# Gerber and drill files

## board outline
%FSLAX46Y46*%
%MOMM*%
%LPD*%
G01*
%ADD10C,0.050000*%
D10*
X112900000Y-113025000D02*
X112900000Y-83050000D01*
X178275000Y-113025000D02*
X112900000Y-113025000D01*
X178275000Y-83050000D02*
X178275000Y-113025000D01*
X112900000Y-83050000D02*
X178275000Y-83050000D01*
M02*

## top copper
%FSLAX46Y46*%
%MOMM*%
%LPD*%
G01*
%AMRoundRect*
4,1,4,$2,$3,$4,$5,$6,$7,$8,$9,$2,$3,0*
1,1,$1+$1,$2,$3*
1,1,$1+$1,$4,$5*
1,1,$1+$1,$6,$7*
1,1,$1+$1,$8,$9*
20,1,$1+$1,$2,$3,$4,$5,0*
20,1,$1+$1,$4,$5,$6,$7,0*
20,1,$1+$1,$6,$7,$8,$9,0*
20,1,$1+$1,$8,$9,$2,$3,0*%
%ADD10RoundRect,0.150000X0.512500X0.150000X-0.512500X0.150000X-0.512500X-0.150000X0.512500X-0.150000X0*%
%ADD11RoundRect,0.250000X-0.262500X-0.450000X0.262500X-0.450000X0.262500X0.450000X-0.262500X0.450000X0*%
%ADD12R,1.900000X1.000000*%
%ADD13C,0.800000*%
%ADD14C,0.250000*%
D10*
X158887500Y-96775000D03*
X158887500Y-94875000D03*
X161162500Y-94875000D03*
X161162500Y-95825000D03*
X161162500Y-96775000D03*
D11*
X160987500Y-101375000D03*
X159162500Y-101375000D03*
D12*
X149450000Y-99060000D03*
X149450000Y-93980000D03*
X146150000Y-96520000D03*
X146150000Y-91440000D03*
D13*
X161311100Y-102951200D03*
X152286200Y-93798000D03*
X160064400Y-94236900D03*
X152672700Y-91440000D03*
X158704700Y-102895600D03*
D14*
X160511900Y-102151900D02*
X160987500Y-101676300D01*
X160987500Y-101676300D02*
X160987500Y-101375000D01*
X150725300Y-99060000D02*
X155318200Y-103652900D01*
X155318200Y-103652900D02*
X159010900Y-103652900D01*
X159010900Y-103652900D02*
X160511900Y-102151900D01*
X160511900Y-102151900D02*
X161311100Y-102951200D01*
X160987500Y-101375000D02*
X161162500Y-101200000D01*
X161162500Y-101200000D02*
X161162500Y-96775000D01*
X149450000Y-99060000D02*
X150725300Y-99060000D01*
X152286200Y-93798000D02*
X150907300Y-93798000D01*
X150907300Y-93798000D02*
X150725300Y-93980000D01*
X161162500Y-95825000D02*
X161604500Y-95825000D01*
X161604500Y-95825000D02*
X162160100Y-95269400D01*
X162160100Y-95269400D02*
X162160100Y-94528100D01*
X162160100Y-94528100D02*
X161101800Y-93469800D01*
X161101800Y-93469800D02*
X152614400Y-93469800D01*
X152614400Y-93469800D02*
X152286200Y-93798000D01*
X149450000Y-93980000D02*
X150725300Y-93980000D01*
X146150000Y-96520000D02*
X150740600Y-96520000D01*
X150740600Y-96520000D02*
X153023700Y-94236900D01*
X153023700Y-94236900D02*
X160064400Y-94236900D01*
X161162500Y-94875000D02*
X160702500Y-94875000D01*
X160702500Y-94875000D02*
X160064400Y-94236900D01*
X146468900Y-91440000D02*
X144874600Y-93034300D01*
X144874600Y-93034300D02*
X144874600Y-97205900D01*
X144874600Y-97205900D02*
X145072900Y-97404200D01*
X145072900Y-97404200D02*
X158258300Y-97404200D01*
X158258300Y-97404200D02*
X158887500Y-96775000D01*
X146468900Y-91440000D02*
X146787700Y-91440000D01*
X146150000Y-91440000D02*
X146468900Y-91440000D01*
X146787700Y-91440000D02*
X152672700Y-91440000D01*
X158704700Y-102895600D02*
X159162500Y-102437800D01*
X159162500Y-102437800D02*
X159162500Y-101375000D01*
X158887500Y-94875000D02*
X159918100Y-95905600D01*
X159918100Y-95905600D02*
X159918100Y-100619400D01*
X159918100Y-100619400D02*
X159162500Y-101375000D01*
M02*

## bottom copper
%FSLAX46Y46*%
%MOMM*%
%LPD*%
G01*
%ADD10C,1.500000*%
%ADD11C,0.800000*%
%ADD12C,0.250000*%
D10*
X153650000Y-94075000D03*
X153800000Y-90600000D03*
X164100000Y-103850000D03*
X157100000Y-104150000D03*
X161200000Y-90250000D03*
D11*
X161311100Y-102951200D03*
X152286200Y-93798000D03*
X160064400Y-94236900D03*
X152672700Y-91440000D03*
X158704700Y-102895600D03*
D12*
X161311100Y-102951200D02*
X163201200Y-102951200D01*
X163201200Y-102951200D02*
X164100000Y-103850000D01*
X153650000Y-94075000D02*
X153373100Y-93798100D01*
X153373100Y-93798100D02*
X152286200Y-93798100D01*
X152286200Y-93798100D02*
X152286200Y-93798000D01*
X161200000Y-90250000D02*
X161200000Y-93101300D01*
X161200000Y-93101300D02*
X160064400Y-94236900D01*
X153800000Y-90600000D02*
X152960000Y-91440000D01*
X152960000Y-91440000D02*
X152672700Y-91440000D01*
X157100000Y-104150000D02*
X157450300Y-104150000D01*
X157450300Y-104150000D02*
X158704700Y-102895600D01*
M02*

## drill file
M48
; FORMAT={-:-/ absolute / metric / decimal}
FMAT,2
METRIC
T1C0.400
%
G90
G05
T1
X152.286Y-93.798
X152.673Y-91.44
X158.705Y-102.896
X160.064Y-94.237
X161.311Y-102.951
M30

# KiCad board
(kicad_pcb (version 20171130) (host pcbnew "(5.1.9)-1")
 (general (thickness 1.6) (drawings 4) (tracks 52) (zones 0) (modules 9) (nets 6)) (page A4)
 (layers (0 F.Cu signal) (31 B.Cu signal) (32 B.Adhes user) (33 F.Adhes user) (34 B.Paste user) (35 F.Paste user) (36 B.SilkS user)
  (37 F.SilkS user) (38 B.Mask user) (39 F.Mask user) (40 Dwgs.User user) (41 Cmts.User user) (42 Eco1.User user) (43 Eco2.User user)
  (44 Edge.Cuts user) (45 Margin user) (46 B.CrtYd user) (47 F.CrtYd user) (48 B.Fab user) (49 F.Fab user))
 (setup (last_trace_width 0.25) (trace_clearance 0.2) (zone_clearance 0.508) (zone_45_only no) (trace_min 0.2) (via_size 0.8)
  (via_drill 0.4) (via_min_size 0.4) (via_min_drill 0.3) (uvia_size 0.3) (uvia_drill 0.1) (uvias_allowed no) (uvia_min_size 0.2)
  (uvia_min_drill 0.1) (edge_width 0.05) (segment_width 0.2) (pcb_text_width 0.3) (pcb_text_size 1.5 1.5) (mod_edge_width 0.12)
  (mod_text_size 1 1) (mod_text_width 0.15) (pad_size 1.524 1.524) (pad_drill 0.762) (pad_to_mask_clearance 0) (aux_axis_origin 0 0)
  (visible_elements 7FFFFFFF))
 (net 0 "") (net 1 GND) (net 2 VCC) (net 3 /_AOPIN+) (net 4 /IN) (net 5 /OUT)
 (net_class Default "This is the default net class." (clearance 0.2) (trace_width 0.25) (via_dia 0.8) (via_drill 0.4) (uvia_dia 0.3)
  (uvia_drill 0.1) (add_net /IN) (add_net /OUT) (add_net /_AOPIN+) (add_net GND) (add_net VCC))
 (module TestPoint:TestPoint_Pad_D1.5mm (layer B.Cu) (at 153.65 94.075)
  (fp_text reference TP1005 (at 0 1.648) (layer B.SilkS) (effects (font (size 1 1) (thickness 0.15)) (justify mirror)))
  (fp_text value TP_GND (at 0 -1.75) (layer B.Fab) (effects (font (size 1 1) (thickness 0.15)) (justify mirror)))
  (pad 1 smd circle (at 0 0) (size 1.5 1.5) (layers B.Cu B.Mask) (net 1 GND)))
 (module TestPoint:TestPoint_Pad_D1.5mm (layer B.Cu) (at 153.8 90.6)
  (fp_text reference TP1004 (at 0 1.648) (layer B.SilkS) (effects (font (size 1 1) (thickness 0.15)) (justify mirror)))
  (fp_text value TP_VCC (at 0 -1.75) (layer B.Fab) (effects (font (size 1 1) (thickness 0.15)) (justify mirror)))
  (pad 1 smd circle (at 0 0) (size 1.5 1.5) (layers B.Cu B.Mask) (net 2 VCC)))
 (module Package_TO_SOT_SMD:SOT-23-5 (layer F.Cu) (at 160.025 95.825 180)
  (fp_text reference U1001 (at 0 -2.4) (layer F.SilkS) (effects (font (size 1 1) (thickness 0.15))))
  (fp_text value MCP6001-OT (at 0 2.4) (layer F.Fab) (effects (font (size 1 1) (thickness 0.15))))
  (pad 5 smd roundrect (at 1.1375 -0.95 180) (size 1.325 0.6) (layers F.Cu F.Paste F.Mask) (roundrect_rratio 0.25) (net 2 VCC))
  (pad 4 smd roundrect (at 1.1375 0.95 180) (size 1.325 0.6) (layers F.Cu F.Paste F.Mask) (roundrect_rratio 0.25) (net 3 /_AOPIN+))
  (pad 3 smd roundrect (at -1.1375 0.95 180) (size 1.325 0.6) (layers F.Cu F.Paste F.Mask) (roundrect_rratio 0.25) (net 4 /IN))
  (pad 2 smd roundrect (at -1.1375 0 180) (size 1.325 0.6) (layers F.Cu F.Paste F.Mask) (roundrect_rratio 0.25) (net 1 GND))
  (pad 1 smd roundrect (at -1.1375 -0.95 180) (size 1.325 0.6) (layers F.Cu F.Paste F.Mask) (roundrect_rratio 0.25) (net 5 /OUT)))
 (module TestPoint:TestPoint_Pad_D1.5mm (layer B.Cu) (at 164.1 103.85 180)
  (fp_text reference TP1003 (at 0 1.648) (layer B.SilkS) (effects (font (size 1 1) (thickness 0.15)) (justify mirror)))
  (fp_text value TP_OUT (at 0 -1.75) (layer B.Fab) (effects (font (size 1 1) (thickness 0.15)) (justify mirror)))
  (pad 1 smd circle (at 0 0 180) (size 1.5 1.5) (layers B.Cu B.Mask) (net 5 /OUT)))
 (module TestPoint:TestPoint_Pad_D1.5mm (layer B.Cu) (at 157.1 104.15)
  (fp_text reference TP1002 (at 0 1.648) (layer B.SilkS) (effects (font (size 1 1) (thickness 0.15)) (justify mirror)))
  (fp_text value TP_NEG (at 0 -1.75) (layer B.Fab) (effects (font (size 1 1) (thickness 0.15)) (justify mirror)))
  (pad 1 smd circle (at 0 0) (size 1.5 1.5) (layers B.Cu B.Mask) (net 3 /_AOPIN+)))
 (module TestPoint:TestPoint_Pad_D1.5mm (layer B.Cu) (at 161.2 90.25)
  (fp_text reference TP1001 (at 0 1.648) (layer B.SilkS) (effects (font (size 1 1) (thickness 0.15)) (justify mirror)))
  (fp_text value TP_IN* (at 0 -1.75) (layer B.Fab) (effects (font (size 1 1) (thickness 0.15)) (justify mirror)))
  (pad 1 smd circle (at 0 0) (size 1.5 1.5) (layers B.Cu B.Mask) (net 4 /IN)))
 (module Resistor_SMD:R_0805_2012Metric (layer F.Cu) (at 160.075 101.375)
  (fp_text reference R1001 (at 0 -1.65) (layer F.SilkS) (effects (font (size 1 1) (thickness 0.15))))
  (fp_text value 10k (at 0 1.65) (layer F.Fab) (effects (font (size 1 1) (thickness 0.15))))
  (pad 2 smd roundrect (at 0.9125 0) (size 1.025 1.4) (layers F.Cu F.Paste F.Mask) (roundrect_rratio 0.243902) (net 5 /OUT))
  (pad 1 smd roundrect (at -0.9125 0) (size 1.025 1.4) (layers F.Cu F.Paste F.Mask) (roundrect_rratio 0.243902) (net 3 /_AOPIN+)))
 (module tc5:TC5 (layer F.Cu) (at 135.3 97.9)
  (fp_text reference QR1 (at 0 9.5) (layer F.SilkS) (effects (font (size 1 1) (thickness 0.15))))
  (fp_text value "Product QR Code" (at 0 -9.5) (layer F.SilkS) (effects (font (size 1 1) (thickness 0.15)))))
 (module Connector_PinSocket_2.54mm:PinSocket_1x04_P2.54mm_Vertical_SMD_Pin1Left (layer F.Cu) (at 147.8 95.25)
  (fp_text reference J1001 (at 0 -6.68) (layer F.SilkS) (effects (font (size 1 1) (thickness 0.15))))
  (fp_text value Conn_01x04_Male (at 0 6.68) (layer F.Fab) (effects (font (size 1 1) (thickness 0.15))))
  (pad 4 smd rect (at 1.65 3.81) (size 1.9 1) (layers F.Cu F.Paste F.Mask) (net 5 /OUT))
  (pad 2 smd rect (at 1.65 -1.27) (size 1.9 1) (layers F.Cu F.Paste F.Mask) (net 1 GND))
  (pad 3 smd rect (at -1.65 1.27) (size 1.9 1) (layers F.Cu F.Paste F.Mask) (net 4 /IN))
  (pad 1 smd rect (at -1.65 -3.81) (size 1.9 1) (layers F.Cu F.Paste F.Mask) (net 2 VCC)))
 (gr_line (start 112.9 113.025) (end 112.9 83.05) (layer Edge.Cuts) (width 0.05))
 (gr_line (start 178.275 113.025) (end 112.9 113.025) (layer Edge.Cuts) (width 0.05))
 (gr_line (start 178.275 83.05) (end 178.275 113.025) (layer Edge.Cuts) (width 0.05))
 (gr_line (start 112.9 83.05) (end 178.275 83.05) (layer Edge.Cuts) (width 0.05))
 (segment (start 160.5119 102.1519) (end 160.9875 101.6763) (width 0.25) (layer F.Cu) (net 5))
 (segment (start 160.9875 101.6763) (end 160.9875 101.375) (width 0.25) (layer F.Cu) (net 5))
 (segment (start 150.7253 99.06) (end 155.3182 103.6529) (width 0.25) (layer F.Cu) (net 5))
 (segment (start 155.3182 103.6529) (end 159.0109 103.6529) (width 0.25) (layer F.Cu) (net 5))
 (segment (start 159.0109 103.6529) (end 160.5119 102.1519) (width 0.25) (layer F.Cu) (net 5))
 (segment (start 160.5119 102.1519) (end 161.3111 102.9512) (width 0.25) (layer F.Cu) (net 5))
 (segment (start 161.3111 102.9512) (end 163.2012 102.9512) (width 0.25) (layer B.Cu) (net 5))
 (segment (start 163.2012 102.9512) (end 164.1 103.85) (width 0.25) (layer B.Cu) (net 5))
 (segment (start 160.9875 101.375) (end 161.1625 101.2) (width 0.25) (layer F.Cu) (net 5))
 (segment (start 161.1625 101.2) (end 161.1625 96.775) (width 0.25) (layer F.Cu) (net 5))
 (segment (start 149.45 99.06) (end 150.7253 99.06) (width 0.25) (layer F.Cu) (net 5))
 (via (at 161.3111 102.9512) (size 0.8) (layers F.Cu B.Cu) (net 5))
 (segment (start 152.2862 93.798) (end 150.9073 93.798) (width 0.25) (layer F.Cu) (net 1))
 (segment (start 150.9073 93.798) (end 150.7253 93.98) (width 0.25) (layer F.Cu) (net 1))
 (segment (start 161.1625 95.825) (end 161.6045 95.825) (width 0.25) (layer F.Cu) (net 1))
 (segment (start 161.6045 95.825) (end 162.1601 95.2694) (width 0.25) (layer F.Cu) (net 1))
 (segment (start 162.1601 95.2694) (end 162.1601 94.5281) (width 0.25) (layer F.Cu) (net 1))
 (segment (start 162.1601 94.5281) (end 161.1018 93.4698) (width 0.25) (layer F.Cu) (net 1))
 (segment (start 161.1018 93.4698) (end 152.6144 93.4698) (width 0.25) (layer F.Cu) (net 1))
 (segment (start 152.6144 93.4698) (end 152.2862 93.798) (width 0.25) (layer F.Cu) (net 1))
 (segment (start 153.65 94.075) (end 153.3731 93.7981) (width 0.25) (layer B.Cu) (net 1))
 (segment (start 153.3731 93.7981) (end 152.2862 93.7981) (width 0.25) (layer B.Cu) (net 1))
 (segment (start 152.2862 93.7981) (end 152.2862 93.798) (width 0.25) (layer B.Cu) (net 1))
 (segment (start 149.45 93.98) (end 150.7253 93.98) (width 0.25) (layer F.Cu) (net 1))
 (via (at 152.2862 93.798) (size 0.8) (layers F.Cu B.Cu) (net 1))
 (segment (start 146.15 96.52) (end 150.7406 96.52) (width 0.25) (layer F.Cu) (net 4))
 (segment (start 150.7406 96.52) (end 153.0237 94.2369) (width 0.25) (layer F.Cu) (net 4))
 (segment (start 153.0237 94.2369) (end 160.0644 94.2369) (width 0.25) (layer F.Cu) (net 4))
 (segment (start 161.1625 94.875) (end 160.7025 94.875) (width 0.25) (layer F.Cu) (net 4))
 (segment (start 160.7025 94.875) (end 160.0644 94.2369) (width 0.25) (layer F.Cu) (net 4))
 (segment (start 161.2 90.25) (end 161.2 93.1013) (width 0.25) (layer B.Cu) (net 4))
 (segment (start 161.2 93.1013) (end 160.0644 94.2369) (width 0.25) (layer B.Cu) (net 4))
 (via (at 160.0644 94.2369) (size 0.8) (layers F.Cu B.Cu) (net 4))
 (segment (start 146.4689 91.44) (end 144.8746 93.0343) (width 0.25) (layer F.Cu) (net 2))
 (segment (start 144.8746 93.0343) (end 144.8746 97.2059) (width 0.25) (layer F.Cu) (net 2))
 (segment (start 144.8746 97.2059) (end 145.0729 97.4042) (width 0.25) (layer F.Cu) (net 2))
 (segment (start 145.0729 97.4042) (end 158.2583 97.4042) (width 0.25) (layer F.Cu) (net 2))
 (segment (start 158.2583 97.4042) (end 158.8875 96.775) (width 0.25) (layer F.Cu) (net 2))
 (segment (start 146.4689 91.44) (end 146.7877 91.44) (width 0.25) (layer F.Cu) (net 2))
 (segment (start 146.15 91.44) (end 146.4689 91.44) (width 0.25) (layer F.Cu) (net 2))
 (segment (start 146.7877 91.44) (end 152.6727 91.44) (width 0.25) (layer F.Cu) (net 2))
 (segment (start 153.8 90.6) (end 152.96 91.44) (width 0.25) (layer B.Cu) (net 2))
 (segment (start 152.96 91.44) (end 152.6727 91.44) (width 0.25) (layer B.Cu) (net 2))
 (via (at 152.6727 91.44) (size 0.8) (layers F.Cu B.Cu) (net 2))
 (segment (start 158.7047 102.8956) (end 159.1625 102.4378) (width 0.25) (layer F.Cu) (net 3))
 (segment (start 159.1625 102.4378) (end 159.1625 101.375) (width 0.25) (layer F.Cu) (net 3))
 (segment (start 157.1 104.15) (end 157.4503 104.15) (width 0.25) (layer B.Cu) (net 3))
 (segment (start 157.4503 104.15) (end 158.7047 102.8956) (width 0.25) (layer B.Cu) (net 3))
 (segment (start 158.8875 94.875) (end 159.9181 95.9056) (width 0.25) (layer F.Cu) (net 3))
 (segment (start 159.9181 95.9056) (end 159.9181 100.6194) (width 0.25) (layer F.Cu) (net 3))
 (segment (start 159.9181 100.6194) (end 159.1625 101.375) (width 0.25) (layer F.Cu) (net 3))
 (via (at 158.7047 102.8956) (size 0.8) (layers F.Cu B.Cu) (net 3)))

